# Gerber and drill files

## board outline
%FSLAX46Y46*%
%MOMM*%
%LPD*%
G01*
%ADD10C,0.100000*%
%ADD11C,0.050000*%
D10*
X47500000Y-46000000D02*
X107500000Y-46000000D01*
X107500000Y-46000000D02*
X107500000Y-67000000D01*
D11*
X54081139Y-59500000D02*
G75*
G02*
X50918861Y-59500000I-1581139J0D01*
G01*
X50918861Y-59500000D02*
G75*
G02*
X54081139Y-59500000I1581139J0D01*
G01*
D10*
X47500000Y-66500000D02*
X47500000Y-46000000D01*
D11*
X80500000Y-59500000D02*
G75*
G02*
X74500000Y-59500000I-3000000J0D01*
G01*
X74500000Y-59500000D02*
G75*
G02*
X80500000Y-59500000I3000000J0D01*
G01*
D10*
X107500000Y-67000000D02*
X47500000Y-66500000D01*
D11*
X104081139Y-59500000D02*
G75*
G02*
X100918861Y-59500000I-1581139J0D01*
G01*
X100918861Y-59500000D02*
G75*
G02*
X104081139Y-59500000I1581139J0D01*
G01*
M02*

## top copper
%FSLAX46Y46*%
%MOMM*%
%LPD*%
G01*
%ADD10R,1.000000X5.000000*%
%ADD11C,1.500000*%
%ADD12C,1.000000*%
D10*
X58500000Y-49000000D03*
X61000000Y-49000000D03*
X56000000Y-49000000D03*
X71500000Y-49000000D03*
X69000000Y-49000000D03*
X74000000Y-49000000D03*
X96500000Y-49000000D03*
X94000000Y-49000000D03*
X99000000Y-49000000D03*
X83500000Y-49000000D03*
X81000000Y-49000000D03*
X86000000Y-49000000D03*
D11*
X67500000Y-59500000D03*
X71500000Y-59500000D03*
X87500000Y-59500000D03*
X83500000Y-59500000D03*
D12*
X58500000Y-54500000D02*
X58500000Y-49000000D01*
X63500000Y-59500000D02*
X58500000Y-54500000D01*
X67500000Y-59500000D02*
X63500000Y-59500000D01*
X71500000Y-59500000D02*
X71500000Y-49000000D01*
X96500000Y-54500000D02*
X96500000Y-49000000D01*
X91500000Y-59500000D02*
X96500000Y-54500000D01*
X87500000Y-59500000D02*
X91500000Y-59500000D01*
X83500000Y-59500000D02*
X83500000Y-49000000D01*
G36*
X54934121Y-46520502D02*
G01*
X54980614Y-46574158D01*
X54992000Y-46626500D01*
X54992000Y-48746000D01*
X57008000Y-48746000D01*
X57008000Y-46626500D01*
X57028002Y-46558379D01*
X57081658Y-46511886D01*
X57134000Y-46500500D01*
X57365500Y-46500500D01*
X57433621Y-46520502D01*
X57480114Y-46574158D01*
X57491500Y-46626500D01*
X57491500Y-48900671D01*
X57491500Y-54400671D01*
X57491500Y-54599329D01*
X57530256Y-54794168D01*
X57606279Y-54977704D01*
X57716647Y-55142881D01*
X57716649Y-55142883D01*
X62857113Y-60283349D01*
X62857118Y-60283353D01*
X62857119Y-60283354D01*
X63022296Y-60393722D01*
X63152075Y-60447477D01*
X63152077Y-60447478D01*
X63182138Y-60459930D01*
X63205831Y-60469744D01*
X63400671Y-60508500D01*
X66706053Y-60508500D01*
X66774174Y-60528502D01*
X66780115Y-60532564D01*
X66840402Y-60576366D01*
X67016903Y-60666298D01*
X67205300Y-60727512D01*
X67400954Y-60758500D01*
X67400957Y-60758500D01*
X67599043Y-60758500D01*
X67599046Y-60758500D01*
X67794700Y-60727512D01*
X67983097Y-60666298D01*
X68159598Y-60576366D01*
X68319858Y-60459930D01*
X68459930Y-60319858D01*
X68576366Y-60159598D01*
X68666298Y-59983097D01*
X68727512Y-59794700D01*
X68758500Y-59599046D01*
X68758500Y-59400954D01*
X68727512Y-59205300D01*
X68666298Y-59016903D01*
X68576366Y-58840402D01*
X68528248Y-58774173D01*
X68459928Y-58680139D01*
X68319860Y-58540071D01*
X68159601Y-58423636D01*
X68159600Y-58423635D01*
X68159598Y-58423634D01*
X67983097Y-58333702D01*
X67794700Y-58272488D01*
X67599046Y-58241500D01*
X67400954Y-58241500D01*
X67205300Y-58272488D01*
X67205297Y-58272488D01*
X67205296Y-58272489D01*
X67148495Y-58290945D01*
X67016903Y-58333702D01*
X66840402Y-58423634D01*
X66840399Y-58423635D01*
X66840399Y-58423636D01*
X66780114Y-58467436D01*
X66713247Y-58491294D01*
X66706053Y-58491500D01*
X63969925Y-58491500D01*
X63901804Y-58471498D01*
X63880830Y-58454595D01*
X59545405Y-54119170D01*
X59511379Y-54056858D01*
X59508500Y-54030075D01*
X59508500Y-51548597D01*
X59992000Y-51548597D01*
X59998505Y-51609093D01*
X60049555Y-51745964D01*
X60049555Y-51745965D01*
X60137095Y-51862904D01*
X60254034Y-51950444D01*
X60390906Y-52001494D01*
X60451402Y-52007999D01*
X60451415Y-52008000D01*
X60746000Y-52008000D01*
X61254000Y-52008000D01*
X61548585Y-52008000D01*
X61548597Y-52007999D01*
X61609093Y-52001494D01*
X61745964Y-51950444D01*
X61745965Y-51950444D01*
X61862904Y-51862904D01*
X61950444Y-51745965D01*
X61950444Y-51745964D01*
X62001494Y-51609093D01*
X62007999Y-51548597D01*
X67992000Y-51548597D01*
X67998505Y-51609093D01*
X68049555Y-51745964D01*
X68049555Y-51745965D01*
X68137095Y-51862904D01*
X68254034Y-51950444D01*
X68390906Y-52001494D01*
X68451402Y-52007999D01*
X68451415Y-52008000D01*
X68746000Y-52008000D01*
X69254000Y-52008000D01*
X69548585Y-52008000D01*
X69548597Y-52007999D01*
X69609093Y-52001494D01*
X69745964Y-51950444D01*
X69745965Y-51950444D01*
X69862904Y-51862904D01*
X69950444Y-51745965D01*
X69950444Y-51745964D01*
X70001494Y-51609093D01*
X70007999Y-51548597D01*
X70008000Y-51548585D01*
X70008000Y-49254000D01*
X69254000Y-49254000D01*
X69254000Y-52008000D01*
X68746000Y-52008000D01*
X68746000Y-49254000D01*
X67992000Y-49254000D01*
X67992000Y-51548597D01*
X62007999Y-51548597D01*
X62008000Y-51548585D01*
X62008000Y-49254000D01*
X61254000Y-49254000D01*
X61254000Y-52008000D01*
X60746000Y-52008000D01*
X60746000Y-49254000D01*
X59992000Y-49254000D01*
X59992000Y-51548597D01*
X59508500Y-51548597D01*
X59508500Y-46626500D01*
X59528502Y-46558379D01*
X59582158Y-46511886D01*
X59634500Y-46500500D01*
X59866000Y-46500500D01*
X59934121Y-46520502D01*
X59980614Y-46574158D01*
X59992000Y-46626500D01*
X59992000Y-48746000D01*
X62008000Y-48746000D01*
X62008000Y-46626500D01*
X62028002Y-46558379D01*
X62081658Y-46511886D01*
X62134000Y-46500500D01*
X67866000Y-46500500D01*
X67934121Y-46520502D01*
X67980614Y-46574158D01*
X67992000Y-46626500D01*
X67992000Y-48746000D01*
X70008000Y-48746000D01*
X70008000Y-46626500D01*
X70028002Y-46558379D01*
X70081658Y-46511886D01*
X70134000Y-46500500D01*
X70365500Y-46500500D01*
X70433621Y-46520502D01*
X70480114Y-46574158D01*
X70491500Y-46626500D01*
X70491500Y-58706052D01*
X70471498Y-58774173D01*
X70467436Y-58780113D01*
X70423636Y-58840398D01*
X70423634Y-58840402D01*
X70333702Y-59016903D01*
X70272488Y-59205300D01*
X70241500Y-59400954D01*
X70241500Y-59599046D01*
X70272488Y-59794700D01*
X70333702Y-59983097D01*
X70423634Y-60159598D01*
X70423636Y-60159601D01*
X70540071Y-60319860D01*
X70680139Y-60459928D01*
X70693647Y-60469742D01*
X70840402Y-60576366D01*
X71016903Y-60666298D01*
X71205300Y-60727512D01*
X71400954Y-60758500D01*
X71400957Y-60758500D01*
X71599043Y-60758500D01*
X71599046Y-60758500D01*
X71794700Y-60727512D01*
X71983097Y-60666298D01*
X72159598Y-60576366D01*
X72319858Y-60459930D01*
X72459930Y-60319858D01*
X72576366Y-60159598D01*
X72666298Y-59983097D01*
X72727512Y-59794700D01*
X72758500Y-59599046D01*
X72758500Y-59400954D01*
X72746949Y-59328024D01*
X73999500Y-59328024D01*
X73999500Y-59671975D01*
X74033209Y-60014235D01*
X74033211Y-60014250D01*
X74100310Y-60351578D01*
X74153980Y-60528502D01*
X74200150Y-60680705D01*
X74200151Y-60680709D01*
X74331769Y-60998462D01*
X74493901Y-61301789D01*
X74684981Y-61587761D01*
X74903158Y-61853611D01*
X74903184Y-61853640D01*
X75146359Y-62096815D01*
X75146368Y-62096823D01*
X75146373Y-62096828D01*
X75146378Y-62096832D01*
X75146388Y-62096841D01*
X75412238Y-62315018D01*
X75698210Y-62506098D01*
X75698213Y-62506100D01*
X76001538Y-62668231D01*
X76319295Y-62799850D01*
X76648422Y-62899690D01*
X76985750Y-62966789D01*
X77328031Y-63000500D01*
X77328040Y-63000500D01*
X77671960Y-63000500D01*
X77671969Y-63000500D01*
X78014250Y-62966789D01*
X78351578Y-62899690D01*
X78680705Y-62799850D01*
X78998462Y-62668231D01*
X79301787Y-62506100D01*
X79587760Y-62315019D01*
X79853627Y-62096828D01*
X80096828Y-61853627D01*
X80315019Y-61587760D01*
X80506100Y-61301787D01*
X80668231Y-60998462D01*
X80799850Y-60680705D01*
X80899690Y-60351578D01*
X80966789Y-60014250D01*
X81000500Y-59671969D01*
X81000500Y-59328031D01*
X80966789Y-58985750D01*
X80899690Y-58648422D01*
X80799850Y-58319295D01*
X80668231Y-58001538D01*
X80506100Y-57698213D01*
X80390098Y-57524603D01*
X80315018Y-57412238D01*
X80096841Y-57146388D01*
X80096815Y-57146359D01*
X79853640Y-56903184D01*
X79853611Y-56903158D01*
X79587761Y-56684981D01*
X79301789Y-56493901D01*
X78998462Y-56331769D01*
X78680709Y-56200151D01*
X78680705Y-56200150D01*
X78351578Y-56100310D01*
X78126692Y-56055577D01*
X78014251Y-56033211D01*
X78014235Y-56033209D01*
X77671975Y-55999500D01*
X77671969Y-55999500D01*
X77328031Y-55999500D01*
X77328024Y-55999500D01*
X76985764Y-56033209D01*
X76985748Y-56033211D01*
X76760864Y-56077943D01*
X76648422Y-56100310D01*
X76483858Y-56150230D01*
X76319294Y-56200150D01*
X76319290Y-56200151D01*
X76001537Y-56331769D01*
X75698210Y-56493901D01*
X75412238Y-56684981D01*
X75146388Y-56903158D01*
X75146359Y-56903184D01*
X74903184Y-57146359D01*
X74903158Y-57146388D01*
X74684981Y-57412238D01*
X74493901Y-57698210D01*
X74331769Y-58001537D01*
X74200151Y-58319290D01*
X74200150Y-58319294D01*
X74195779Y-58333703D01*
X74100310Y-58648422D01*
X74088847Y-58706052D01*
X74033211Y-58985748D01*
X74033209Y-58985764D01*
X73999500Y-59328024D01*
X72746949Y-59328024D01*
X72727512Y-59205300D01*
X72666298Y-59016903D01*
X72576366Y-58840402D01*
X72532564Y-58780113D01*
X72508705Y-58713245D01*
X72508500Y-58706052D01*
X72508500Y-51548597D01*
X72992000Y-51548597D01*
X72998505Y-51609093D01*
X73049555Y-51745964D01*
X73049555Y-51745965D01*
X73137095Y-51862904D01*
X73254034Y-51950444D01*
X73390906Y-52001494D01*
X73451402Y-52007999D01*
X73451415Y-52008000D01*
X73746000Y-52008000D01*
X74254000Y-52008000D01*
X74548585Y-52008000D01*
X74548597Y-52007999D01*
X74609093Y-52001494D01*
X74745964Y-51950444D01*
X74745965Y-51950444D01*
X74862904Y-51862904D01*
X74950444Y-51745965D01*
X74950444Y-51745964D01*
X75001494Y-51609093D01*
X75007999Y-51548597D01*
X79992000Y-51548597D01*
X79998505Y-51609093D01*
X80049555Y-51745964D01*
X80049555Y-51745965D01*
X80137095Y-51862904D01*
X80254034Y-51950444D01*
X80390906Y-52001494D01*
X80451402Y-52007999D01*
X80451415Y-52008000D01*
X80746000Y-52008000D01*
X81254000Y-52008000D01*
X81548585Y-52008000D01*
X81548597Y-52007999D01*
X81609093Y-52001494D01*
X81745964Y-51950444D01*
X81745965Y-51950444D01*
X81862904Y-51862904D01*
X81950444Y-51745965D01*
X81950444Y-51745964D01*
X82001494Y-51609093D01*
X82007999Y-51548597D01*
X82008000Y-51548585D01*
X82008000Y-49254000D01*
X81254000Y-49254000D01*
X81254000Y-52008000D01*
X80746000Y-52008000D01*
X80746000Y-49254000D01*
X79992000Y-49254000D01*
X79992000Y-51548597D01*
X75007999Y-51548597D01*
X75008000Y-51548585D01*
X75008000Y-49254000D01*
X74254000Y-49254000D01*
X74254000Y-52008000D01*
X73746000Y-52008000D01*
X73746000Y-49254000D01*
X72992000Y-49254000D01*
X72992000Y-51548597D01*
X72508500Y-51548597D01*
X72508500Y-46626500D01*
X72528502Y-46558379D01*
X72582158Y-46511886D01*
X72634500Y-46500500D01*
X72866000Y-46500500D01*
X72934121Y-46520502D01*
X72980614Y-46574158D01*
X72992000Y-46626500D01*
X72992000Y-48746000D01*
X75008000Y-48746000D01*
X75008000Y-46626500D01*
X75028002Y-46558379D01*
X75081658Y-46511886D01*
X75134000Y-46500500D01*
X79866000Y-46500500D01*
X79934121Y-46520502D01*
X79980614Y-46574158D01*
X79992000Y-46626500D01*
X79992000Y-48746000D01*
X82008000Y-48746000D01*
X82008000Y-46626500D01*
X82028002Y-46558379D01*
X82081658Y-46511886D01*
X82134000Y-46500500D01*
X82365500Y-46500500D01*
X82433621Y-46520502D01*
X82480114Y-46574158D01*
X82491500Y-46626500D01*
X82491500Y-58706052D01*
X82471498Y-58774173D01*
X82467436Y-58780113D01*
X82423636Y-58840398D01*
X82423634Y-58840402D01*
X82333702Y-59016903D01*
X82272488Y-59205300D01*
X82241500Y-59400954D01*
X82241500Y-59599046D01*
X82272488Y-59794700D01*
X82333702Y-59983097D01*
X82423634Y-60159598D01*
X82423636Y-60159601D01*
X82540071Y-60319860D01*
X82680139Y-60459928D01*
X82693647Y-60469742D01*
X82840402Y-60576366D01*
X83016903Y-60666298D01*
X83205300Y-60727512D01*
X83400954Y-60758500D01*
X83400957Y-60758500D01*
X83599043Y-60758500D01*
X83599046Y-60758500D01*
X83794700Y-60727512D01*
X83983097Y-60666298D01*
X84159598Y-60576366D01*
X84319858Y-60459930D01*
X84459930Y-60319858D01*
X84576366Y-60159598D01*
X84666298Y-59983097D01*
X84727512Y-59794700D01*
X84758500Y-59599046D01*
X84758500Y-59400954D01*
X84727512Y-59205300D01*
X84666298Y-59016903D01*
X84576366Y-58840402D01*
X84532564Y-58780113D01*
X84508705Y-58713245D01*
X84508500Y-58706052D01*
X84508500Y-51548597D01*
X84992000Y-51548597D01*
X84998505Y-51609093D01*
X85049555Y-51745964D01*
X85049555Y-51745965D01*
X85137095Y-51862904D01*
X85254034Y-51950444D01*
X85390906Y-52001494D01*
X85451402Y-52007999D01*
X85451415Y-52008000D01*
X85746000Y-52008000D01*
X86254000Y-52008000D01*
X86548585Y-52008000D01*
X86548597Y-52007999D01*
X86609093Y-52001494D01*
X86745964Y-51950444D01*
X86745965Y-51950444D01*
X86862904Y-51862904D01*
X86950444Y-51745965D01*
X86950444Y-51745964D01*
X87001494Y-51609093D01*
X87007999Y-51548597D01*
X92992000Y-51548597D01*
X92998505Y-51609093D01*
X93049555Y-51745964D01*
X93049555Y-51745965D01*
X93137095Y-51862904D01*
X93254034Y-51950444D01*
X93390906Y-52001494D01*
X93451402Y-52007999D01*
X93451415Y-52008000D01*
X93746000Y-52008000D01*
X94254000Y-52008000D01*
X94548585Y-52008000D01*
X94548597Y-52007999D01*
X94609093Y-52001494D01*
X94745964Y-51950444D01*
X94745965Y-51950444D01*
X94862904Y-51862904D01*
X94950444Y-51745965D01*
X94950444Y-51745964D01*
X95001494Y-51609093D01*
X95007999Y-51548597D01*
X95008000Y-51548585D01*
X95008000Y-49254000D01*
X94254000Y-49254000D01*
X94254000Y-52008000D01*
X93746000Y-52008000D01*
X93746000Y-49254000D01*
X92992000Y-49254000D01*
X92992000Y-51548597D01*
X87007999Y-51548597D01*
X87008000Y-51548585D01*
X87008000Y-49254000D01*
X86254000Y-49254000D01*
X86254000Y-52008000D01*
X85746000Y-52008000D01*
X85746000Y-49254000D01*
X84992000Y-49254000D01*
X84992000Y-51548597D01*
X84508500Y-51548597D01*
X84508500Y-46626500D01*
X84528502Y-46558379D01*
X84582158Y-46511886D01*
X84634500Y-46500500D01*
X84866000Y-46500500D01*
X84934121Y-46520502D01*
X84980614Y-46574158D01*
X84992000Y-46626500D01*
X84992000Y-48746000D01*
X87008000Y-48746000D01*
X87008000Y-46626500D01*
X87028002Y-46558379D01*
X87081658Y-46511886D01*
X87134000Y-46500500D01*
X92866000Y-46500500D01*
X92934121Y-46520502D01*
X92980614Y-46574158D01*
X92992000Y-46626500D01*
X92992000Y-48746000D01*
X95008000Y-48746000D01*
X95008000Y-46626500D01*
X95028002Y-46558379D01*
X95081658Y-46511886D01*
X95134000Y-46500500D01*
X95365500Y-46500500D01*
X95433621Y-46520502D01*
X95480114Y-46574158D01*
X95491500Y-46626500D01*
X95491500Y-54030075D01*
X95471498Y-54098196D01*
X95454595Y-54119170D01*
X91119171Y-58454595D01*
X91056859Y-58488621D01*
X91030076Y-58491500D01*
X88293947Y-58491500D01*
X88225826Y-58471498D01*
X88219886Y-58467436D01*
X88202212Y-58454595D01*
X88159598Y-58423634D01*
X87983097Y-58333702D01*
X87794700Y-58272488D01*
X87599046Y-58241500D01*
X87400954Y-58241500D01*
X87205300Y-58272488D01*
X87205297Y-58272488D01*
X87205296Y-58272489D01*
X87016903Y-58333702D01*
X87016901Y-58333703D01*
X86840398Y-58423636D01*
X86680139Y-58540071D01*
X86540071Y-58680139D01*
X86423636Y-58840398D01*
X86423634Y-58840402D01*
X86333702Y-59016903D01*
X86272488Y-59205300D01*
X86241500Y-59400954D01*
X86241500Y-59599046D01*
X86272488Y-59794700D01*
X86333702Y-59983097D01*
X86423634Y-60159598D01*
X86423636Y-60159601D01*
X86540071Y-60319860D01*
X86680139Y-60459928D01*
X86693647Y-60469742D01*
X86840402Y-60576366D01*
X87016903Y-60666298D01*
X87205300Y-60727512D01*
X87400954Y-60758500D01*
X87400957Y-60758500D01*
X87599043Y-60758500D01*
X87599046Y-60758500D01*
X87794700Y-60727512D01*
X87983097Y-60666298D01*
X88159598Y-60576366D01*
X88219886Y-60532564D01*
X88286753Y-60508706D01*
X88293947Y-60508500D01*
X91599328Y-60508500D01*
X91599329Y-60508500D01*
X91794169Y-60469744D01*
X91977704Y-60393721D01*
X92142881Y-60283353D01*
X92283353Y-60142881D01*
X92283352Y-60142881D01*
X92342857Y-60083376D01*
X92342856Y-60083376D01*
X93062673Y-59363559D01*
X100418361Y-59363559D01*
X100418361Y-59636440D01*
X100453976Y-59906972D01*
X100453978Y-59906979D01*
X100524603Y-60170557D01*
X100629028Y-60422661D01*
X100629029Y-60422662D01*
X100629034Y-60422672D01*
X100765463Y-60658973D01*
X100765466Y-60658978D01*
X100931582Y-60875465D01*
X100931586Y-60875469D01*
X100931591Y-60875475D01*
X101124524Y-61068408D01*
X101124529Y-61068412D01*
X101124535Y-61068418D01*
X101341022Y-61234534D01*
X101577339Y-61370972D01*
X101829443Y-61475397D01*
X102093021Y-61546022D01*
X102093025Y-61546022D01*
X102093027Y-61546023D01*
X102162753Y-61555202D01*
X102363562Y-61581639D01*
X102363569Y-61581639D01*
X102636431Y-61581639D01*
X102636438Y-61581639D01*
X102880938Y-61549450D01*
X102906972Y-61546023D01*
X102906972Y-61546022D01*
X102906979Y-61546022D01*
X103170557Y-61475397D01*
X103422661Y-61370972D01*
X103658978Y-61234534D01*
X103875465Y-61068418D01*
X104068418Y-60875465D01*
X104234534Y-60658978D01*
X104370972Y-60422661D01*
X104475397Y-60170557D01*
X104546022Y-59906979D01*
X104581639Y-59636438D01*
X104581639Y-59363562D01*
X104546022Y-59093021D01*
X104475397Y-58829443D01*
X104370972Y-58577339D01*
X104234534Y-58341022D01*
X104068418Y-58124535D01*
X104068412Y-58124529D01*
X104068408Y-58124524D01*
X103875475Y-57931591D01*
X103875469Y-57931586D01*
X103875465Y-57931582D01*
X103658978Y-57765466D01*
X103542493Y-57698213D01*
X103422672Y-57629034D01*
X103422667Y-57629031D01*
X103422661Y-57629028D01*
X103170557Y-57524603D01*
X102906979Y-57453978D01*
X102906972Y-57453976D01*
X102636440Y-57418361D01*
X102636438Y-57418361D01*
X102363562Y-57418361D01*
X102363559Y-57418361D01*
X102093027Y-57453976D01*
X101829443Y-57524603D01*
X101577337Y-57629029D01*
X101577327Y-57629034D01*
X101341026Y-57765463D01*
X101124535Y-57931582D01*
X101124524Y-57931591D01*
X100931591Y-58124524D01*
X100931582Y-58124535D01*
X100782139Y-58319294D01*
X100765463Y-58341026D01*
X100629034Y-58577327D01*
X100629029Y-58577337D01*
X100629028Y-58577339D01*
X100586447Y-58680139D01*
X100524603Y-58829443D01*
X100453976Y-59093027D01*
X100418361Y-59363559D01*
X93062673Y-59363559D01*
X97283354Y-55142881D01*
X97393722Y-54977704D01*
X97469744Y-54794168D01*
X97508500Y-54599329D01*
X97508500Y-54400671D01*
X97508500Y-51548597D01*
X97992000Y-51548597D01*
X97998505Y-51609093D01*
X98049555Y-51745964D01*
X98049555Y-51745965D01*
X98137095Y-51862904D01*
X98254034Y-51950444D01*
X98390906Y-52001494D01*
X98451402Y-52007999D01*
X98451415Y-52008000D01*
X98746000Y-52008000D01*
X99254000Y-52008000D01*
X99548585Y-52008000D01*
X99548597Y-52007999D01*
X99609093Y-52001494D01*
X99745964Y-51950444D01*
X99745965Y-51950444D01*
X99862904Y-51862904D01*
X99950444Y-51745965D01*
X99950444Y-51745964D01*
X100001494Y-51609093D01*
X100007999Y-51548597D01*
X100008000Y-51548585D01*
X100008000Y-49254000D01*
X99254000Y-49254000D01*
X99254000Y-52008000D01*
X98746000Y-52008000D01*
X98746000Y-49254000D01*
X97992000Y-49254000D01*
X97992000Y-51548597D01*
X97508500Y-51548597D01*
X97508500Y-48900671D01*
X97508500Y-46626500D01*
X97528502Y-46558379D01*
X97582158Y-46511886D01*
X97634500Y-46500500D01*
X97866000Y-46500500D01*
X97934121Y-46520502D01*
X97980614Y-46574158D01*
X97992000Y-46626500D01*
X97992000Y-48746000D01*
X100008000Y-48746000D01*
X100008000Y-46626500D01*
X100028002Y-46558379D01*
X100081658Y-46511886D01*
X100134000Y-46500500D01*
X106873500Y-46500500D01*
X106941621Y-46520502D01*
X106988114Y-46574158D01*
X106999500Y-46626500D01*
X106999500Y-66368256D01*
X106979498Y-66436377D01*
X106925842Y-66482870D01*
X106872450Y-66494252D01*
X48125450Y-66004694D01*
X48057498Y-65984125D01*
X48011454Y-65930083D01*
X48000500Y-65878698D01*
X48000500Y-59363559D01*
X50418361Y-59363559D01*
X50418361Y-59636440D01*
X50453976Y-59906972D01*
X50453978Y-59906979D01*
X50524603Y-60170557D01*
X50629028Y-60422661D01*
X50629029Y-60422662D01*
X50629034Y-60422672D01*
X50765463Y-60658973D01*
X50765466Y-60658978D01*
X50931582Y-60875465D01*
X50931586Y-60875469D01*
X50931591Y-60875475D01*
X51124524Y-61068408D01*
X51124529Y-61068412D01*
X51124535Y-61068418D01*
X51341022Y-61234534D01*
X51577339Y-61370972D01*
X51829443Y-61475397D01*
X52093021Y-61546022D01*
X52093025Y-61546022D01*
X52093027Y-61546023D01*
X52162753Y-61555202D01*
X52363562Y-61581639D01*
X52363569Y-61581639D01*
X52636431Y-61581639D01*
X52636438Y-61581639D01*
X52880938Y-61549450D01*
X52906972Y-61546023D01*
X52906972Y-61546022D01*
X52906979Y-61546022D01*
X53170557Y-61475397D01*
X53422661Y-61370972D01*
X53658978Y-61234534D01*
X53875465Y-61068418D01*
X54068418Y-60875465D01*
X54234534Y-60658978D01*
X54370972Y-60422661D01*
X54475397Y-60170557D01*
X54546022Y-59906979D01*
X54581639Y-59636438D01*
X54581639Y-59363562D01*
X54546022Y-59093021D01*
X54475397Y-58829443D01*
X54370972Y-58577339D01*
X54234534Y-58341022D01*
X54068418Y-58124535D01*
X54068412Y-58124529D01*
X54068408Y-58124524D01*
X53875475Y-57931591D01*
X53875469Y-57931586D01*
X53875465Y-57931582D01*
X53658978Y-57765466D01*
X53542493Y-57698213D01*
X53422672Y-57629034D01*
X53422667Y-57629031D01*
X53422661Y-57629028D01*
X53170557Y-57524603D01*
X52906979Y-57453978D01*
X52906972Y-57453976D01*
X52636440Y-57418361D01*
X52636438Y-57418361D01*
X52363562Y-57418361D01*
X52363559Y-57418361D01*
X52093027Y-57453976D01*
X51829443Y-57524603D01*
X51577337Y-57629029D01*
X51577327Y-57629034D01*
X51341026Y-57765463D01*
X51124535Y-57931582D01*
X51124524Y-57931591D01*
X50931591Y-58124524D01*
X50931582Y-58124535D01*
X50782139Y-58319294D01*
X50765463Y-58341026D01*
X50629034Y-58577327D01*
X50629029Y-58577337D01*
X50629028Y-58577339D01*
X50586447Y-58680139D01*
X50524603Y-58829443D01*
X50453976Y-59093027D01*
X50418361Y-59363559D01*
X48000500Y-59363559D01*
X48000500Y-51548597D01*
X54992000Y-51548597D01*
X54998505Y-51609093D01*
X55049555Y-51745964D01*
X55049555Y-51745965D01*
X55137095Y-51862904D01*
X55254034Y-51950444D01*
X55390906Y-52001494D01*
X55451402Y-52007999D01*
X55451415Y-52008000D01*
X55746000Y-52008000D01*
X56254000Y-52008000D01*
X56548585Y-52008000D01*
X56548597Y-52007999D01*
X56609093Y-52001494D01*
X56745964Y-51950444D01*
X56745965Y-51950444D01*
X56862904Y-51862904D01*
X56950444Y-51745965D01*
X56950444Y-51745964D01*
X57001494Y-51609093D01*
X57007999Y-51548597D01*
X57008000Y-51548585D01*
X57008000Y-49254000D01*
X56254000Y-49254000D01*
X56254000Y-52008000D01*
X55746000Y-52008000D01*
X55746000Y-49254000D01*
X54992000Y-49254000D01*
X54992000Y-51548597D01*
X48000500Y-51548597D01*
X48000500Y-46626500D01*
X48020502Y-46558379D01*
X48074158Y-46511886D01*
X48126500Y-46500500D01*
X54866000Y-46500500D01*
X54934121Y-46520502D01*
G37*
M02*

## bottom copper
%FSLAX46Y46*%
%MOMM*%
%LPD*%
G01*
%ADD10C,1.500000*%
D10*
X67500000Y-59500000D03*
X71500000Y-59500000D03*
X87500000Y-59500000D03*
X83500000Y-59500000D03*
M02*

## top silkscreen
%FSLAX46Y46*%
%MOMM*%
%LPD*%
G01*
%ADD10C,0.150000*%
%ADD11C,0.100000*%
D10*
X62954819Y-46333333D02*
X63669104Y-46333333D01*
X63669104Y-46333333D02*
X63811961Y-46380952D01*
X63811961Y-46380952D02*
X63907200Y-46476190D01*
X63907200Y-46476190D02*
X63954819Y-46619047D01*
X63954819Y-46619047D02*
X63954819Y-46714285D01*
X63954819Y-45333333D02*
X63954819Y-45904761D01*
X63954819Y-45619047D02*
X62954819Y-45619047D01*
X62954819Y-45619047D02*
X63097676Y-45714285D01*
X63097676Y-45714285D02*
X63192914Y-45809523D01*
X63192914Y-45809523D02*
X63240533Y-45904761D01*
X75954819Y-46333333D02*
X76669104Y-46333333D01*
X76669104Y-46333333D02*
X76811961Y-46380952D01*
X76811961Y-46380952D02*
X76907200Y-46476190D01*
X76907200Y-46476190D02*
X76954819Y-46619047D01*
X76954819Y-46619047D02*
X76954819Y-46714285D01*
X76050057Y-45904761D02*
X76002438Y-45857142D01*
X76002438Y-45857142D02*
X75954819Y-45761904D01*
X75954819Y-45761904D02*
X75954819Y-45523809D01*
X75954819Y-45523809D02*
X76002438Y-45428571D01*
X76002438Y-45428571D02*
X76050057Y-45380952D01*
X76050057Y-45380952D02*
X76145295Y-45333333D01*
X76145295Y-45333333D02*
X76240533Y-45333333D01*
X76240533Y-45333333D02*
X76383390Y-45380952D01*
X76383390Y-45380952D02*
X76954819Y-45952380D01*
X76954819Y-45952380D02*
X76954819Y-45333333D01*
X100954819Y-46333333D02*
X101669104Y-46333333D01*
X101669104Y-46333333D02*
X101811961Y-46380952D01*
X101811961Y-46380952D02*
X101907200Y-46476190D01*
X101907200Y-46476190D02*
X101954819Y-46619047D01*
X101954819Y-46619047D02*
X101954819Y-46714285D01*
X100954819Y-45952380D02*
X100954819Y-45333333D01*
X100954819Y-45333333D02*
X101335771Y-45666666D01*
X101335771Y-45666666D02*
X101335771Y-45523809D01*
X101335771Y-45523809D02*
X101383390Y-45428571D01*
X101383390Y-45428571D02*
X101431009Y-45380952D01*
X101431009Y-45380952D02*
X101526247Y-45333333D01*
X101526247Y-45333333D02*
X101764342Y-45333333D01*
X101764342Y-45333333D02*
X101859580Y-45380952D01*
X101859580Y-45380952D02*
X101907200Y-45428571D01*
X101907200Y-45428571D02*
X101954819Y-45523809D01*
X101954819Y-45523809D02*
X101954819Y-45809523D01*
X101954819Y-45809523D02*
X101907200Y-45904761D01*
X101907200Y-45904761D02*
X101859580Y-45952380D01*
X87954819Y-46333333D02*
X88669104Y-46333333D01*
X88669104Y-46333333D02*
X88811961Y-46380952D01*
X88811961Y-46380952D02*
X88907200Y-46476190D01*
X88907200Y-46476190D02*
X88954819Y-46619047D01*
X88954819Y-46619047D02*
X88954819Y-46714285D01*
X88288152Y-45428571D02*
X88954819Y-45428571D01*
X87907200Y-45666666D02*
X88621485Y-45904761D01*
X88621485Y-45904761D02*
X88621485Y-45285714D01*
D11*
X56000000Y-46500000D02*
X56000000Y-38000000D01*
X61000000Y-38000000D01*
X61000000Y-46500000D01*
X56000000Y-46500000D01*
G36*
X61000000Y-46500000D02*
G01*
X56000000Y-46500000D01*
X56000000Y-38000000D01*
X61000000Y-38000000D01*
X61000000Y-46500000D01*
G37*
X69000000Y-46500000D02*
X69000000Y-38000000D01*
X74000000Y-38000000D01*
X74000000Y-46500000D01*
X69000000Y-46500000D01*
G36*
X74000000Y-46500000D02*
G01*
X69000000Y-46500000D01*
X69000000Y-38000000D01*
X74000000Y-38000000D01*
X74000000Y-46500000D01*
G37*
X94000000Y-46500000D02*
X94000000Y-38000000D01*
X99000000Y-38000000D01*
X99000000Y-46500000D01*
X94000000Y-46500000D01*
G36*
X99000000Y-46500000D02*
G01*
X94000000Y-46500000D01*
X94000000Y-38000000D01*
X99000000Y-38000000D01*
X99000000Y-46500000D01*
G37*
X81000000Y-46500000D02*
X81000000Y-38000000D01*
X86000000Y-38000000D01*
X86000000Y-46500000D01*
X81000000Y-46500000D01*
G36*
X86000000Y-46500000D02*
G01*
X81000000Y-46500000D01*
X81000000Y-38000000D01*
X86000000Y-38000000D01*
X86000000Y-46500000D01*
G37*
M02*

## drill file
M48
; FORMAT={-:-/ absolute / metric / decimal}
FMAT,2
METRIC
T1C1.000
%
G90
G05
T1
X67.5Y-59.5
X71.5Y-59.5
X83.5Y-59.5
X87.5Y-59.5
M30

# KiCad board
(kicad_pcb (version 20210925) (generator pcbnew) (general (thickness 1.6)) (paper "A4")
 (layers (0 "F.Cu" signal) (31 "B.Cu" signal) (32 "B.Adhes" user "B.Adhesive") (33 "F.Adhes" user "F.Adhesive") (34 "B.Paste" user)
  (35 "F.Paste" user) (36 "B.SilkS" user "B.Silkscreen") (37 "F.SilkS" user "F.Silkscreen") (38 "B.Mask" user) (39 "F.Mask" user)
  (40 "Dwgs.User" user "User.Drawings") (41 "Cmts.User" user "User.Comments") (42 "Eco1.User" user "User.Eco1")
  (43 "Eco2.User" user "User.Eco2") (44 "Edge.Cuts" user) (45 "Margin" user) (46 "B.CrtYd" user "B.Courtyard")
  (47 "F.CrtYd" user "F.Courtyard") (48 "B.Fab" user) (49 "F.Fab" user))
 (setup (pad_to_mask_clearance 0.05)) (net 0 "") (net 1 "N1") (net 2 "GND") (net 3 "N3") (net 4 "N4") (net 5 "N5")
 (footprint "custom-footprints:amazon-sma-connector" (layer "F.Cu") (at 64 46 -90)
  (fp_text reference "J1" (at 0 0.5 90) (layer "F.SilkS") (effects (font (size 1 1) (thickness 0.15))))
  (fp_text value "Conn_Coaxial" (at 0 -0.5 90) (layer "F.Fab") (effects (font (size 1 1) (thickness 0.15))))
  (fp_poly (pts (xy 0.5 8) (xy -8 8) (xy -8 3) (xy 0.5 3)) (layer "F.SilkS") (width 0.1) (fill solid))
  (pad "1" connect rect locked (at 3 5.5 270) (size 5 1) (layers "F.Cu" "F.Mask") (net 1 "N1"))
  (pad "2" connect rect locked (at 3 3 270) (size 5 1) (layers "F.Cu" "F.Mask") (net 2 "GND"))
  (pad "2" connect rect locked (at 3 8 270) (size 5 1) (layers "F.Cu" "F.Mask") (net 2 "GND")))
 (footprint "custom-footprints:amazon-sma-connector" (layer "F.Cu") (at 77 46 -90)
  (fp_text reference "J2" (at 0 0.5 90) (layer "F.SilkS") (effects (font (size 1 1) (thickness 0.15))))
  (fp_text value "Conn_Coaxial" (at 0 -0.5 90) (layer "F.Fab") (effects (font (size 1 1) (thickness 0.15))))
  (fp_poly (pts (xy 0.5 8) (xy -8 8) (xy -8 3) (xy 0.5 3)) (layer "F.SilkS") (width 0.1) (fill solid))
  (pad "1" connect rect locked (at 3 5.5 270) (size 5 1) (layers "F.Cu" "F.Mask") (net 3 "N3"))
  (pad "2" connect rect locked (at 3 8 270) (size 5 1) (layers "F.Cu" "F.Mask") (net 2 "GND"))
  (pad "2" connect rect locked (at 3 3 270) (size 5 1) (layers "F.Cu" "F.Mask") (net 2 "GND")))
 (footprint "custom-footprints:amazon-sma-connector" (layer "F.Cu") (at 102 46 -90)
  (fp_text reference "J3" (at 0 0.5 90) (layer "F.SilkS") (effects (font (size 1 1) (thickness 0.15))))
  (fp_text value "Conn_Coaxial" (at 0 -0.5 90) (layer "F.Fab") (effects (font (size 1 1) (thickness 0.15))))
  (fp_poly (pts (xy 0.5 8) (xy -8 8) (xy -8 3) (xy 0.5 3)) (layer "F.SilkS") (width 0.1) (fill solid))
  (pad "1" connect rect locked (at 3 5.5 270) (size 5 1) (layers "F.Cu" "F.Mask") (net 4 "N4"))
  (pad "2" connect rect locked (at 3 8 270) (size 5 1) (layers "F.Cu" "F.Mask") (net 2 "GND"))
  (pad "2" connect rect locked (at 3 3 270) (size 5 1) (layers "F.Cu" "F.Mask") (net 2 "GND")))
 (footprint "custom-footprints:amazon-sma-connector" (layer "F.Cu") (at 89 46 -90)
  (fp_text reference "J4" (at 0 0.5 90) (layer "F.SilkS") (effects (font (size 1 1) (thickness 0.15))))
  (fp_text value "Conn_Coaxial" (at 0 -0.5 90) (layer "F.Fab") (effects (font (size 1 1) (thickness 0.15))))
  (fp_poly (pts (xy 0.5 8) (xy -8 8) (xy -8 3) (xy 0.5 3)) (layer "F.SilkS") (width 0.1) (fill solid))
  (pad "1" connect rect locked (at 3 5.5 270) (size 5 1) (layers "F.Cu" "F.Mask") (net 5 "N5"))
  (pad "2" connect rect locked (at 3 8 270) (size 5 1) (layers "F.Cu" "F.Mask") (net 2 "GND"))
  (pad "2" connect rect locked (at 3 3 270) (size 5 1) (layers "F.Cu" "F.Mask") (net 2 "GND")))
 (gr_line (start 47.5 46) (end 107.5 46) (layer "Edge.Cuts") (width 0.1))
 (gr_line (start 107.5 46) (end 107.5 67) (layer "Edge.Cuts") (width 0.1))
 (gr_circle (center 52.5 59.5) (end 54 60) (layer "Edge.Cuts") (width 0.05) (fill none))
 (gr_line (start 47.5 66.5) (end 47.5 46) (layer "Edge.Cuts") (width 0.1))
 (gr_circle (center 77.5 59.5) (end 80.5 59.5) (layer "Edge.Cuts") (width 0.05) (fill none))
 (gr_line (start 107.5 67) (end 47.5 66.5) (layer "Edge.Cuts") (width 0.1))
 (gr_circle (center 102.5 59.5) (end 104 60) (layer "Edge.Cuts") (width 0.05) (fill none))
 (segment (start 58.5 54.5) (end 58.5 49) (width 1) (layer "F.Cu") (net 1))
 (segment (start 63.5 59.5) (end 58.5 54.5) (width 1) (layer "F.Cu") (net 1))
 (segment (start 67.5 59.5) (end 63.5 59.5) (width 1) (layer "F.Cu") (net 1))
 (via (at 67.5 59.5) (size 1.5) (drill 1) (layers "F.Cu" "B.Cu") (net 1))
 (segment (start 71.5 59.5) (end 71.5 49) (width 1) (layer "F.Cu") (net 3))
 (via (at 71.5 59.5) (size 1.5) (drill 1) (layers "F.Cu" "B.Cu") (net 3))
 (segment (start 96.5 54.5) (end 96.5 49) (width 1) (layer "F.Cu") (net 4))
 (segment (start 91.5 59.5) (end 96.5 54.5) (width 1) (layer "F.Cu") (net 4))
 (segment (start 87.5 59.5) (end 91.5 59.5) (width 1) (layer "F.Cu") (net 4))
 (via (at 87.5 59.5) (size 1.5) (drill 1) (layers "F.Cu" "B.Cu") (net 4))
 (segment (start 83.5 59.5) (end 83.5 49) (width 1) (layer "F.Cu") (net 5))
 (via (at 83.5 59.5) (size 1.5) (drill 1) (layers "F.Cu" "B.Cu") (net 5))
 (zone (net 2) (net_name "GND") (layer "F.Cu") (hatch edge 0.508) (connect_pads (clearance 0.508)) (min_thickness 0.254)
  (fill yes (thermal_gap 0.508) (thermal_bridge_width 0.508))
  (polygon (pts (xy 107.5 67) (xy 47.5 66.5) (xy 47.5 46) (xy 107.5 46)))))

